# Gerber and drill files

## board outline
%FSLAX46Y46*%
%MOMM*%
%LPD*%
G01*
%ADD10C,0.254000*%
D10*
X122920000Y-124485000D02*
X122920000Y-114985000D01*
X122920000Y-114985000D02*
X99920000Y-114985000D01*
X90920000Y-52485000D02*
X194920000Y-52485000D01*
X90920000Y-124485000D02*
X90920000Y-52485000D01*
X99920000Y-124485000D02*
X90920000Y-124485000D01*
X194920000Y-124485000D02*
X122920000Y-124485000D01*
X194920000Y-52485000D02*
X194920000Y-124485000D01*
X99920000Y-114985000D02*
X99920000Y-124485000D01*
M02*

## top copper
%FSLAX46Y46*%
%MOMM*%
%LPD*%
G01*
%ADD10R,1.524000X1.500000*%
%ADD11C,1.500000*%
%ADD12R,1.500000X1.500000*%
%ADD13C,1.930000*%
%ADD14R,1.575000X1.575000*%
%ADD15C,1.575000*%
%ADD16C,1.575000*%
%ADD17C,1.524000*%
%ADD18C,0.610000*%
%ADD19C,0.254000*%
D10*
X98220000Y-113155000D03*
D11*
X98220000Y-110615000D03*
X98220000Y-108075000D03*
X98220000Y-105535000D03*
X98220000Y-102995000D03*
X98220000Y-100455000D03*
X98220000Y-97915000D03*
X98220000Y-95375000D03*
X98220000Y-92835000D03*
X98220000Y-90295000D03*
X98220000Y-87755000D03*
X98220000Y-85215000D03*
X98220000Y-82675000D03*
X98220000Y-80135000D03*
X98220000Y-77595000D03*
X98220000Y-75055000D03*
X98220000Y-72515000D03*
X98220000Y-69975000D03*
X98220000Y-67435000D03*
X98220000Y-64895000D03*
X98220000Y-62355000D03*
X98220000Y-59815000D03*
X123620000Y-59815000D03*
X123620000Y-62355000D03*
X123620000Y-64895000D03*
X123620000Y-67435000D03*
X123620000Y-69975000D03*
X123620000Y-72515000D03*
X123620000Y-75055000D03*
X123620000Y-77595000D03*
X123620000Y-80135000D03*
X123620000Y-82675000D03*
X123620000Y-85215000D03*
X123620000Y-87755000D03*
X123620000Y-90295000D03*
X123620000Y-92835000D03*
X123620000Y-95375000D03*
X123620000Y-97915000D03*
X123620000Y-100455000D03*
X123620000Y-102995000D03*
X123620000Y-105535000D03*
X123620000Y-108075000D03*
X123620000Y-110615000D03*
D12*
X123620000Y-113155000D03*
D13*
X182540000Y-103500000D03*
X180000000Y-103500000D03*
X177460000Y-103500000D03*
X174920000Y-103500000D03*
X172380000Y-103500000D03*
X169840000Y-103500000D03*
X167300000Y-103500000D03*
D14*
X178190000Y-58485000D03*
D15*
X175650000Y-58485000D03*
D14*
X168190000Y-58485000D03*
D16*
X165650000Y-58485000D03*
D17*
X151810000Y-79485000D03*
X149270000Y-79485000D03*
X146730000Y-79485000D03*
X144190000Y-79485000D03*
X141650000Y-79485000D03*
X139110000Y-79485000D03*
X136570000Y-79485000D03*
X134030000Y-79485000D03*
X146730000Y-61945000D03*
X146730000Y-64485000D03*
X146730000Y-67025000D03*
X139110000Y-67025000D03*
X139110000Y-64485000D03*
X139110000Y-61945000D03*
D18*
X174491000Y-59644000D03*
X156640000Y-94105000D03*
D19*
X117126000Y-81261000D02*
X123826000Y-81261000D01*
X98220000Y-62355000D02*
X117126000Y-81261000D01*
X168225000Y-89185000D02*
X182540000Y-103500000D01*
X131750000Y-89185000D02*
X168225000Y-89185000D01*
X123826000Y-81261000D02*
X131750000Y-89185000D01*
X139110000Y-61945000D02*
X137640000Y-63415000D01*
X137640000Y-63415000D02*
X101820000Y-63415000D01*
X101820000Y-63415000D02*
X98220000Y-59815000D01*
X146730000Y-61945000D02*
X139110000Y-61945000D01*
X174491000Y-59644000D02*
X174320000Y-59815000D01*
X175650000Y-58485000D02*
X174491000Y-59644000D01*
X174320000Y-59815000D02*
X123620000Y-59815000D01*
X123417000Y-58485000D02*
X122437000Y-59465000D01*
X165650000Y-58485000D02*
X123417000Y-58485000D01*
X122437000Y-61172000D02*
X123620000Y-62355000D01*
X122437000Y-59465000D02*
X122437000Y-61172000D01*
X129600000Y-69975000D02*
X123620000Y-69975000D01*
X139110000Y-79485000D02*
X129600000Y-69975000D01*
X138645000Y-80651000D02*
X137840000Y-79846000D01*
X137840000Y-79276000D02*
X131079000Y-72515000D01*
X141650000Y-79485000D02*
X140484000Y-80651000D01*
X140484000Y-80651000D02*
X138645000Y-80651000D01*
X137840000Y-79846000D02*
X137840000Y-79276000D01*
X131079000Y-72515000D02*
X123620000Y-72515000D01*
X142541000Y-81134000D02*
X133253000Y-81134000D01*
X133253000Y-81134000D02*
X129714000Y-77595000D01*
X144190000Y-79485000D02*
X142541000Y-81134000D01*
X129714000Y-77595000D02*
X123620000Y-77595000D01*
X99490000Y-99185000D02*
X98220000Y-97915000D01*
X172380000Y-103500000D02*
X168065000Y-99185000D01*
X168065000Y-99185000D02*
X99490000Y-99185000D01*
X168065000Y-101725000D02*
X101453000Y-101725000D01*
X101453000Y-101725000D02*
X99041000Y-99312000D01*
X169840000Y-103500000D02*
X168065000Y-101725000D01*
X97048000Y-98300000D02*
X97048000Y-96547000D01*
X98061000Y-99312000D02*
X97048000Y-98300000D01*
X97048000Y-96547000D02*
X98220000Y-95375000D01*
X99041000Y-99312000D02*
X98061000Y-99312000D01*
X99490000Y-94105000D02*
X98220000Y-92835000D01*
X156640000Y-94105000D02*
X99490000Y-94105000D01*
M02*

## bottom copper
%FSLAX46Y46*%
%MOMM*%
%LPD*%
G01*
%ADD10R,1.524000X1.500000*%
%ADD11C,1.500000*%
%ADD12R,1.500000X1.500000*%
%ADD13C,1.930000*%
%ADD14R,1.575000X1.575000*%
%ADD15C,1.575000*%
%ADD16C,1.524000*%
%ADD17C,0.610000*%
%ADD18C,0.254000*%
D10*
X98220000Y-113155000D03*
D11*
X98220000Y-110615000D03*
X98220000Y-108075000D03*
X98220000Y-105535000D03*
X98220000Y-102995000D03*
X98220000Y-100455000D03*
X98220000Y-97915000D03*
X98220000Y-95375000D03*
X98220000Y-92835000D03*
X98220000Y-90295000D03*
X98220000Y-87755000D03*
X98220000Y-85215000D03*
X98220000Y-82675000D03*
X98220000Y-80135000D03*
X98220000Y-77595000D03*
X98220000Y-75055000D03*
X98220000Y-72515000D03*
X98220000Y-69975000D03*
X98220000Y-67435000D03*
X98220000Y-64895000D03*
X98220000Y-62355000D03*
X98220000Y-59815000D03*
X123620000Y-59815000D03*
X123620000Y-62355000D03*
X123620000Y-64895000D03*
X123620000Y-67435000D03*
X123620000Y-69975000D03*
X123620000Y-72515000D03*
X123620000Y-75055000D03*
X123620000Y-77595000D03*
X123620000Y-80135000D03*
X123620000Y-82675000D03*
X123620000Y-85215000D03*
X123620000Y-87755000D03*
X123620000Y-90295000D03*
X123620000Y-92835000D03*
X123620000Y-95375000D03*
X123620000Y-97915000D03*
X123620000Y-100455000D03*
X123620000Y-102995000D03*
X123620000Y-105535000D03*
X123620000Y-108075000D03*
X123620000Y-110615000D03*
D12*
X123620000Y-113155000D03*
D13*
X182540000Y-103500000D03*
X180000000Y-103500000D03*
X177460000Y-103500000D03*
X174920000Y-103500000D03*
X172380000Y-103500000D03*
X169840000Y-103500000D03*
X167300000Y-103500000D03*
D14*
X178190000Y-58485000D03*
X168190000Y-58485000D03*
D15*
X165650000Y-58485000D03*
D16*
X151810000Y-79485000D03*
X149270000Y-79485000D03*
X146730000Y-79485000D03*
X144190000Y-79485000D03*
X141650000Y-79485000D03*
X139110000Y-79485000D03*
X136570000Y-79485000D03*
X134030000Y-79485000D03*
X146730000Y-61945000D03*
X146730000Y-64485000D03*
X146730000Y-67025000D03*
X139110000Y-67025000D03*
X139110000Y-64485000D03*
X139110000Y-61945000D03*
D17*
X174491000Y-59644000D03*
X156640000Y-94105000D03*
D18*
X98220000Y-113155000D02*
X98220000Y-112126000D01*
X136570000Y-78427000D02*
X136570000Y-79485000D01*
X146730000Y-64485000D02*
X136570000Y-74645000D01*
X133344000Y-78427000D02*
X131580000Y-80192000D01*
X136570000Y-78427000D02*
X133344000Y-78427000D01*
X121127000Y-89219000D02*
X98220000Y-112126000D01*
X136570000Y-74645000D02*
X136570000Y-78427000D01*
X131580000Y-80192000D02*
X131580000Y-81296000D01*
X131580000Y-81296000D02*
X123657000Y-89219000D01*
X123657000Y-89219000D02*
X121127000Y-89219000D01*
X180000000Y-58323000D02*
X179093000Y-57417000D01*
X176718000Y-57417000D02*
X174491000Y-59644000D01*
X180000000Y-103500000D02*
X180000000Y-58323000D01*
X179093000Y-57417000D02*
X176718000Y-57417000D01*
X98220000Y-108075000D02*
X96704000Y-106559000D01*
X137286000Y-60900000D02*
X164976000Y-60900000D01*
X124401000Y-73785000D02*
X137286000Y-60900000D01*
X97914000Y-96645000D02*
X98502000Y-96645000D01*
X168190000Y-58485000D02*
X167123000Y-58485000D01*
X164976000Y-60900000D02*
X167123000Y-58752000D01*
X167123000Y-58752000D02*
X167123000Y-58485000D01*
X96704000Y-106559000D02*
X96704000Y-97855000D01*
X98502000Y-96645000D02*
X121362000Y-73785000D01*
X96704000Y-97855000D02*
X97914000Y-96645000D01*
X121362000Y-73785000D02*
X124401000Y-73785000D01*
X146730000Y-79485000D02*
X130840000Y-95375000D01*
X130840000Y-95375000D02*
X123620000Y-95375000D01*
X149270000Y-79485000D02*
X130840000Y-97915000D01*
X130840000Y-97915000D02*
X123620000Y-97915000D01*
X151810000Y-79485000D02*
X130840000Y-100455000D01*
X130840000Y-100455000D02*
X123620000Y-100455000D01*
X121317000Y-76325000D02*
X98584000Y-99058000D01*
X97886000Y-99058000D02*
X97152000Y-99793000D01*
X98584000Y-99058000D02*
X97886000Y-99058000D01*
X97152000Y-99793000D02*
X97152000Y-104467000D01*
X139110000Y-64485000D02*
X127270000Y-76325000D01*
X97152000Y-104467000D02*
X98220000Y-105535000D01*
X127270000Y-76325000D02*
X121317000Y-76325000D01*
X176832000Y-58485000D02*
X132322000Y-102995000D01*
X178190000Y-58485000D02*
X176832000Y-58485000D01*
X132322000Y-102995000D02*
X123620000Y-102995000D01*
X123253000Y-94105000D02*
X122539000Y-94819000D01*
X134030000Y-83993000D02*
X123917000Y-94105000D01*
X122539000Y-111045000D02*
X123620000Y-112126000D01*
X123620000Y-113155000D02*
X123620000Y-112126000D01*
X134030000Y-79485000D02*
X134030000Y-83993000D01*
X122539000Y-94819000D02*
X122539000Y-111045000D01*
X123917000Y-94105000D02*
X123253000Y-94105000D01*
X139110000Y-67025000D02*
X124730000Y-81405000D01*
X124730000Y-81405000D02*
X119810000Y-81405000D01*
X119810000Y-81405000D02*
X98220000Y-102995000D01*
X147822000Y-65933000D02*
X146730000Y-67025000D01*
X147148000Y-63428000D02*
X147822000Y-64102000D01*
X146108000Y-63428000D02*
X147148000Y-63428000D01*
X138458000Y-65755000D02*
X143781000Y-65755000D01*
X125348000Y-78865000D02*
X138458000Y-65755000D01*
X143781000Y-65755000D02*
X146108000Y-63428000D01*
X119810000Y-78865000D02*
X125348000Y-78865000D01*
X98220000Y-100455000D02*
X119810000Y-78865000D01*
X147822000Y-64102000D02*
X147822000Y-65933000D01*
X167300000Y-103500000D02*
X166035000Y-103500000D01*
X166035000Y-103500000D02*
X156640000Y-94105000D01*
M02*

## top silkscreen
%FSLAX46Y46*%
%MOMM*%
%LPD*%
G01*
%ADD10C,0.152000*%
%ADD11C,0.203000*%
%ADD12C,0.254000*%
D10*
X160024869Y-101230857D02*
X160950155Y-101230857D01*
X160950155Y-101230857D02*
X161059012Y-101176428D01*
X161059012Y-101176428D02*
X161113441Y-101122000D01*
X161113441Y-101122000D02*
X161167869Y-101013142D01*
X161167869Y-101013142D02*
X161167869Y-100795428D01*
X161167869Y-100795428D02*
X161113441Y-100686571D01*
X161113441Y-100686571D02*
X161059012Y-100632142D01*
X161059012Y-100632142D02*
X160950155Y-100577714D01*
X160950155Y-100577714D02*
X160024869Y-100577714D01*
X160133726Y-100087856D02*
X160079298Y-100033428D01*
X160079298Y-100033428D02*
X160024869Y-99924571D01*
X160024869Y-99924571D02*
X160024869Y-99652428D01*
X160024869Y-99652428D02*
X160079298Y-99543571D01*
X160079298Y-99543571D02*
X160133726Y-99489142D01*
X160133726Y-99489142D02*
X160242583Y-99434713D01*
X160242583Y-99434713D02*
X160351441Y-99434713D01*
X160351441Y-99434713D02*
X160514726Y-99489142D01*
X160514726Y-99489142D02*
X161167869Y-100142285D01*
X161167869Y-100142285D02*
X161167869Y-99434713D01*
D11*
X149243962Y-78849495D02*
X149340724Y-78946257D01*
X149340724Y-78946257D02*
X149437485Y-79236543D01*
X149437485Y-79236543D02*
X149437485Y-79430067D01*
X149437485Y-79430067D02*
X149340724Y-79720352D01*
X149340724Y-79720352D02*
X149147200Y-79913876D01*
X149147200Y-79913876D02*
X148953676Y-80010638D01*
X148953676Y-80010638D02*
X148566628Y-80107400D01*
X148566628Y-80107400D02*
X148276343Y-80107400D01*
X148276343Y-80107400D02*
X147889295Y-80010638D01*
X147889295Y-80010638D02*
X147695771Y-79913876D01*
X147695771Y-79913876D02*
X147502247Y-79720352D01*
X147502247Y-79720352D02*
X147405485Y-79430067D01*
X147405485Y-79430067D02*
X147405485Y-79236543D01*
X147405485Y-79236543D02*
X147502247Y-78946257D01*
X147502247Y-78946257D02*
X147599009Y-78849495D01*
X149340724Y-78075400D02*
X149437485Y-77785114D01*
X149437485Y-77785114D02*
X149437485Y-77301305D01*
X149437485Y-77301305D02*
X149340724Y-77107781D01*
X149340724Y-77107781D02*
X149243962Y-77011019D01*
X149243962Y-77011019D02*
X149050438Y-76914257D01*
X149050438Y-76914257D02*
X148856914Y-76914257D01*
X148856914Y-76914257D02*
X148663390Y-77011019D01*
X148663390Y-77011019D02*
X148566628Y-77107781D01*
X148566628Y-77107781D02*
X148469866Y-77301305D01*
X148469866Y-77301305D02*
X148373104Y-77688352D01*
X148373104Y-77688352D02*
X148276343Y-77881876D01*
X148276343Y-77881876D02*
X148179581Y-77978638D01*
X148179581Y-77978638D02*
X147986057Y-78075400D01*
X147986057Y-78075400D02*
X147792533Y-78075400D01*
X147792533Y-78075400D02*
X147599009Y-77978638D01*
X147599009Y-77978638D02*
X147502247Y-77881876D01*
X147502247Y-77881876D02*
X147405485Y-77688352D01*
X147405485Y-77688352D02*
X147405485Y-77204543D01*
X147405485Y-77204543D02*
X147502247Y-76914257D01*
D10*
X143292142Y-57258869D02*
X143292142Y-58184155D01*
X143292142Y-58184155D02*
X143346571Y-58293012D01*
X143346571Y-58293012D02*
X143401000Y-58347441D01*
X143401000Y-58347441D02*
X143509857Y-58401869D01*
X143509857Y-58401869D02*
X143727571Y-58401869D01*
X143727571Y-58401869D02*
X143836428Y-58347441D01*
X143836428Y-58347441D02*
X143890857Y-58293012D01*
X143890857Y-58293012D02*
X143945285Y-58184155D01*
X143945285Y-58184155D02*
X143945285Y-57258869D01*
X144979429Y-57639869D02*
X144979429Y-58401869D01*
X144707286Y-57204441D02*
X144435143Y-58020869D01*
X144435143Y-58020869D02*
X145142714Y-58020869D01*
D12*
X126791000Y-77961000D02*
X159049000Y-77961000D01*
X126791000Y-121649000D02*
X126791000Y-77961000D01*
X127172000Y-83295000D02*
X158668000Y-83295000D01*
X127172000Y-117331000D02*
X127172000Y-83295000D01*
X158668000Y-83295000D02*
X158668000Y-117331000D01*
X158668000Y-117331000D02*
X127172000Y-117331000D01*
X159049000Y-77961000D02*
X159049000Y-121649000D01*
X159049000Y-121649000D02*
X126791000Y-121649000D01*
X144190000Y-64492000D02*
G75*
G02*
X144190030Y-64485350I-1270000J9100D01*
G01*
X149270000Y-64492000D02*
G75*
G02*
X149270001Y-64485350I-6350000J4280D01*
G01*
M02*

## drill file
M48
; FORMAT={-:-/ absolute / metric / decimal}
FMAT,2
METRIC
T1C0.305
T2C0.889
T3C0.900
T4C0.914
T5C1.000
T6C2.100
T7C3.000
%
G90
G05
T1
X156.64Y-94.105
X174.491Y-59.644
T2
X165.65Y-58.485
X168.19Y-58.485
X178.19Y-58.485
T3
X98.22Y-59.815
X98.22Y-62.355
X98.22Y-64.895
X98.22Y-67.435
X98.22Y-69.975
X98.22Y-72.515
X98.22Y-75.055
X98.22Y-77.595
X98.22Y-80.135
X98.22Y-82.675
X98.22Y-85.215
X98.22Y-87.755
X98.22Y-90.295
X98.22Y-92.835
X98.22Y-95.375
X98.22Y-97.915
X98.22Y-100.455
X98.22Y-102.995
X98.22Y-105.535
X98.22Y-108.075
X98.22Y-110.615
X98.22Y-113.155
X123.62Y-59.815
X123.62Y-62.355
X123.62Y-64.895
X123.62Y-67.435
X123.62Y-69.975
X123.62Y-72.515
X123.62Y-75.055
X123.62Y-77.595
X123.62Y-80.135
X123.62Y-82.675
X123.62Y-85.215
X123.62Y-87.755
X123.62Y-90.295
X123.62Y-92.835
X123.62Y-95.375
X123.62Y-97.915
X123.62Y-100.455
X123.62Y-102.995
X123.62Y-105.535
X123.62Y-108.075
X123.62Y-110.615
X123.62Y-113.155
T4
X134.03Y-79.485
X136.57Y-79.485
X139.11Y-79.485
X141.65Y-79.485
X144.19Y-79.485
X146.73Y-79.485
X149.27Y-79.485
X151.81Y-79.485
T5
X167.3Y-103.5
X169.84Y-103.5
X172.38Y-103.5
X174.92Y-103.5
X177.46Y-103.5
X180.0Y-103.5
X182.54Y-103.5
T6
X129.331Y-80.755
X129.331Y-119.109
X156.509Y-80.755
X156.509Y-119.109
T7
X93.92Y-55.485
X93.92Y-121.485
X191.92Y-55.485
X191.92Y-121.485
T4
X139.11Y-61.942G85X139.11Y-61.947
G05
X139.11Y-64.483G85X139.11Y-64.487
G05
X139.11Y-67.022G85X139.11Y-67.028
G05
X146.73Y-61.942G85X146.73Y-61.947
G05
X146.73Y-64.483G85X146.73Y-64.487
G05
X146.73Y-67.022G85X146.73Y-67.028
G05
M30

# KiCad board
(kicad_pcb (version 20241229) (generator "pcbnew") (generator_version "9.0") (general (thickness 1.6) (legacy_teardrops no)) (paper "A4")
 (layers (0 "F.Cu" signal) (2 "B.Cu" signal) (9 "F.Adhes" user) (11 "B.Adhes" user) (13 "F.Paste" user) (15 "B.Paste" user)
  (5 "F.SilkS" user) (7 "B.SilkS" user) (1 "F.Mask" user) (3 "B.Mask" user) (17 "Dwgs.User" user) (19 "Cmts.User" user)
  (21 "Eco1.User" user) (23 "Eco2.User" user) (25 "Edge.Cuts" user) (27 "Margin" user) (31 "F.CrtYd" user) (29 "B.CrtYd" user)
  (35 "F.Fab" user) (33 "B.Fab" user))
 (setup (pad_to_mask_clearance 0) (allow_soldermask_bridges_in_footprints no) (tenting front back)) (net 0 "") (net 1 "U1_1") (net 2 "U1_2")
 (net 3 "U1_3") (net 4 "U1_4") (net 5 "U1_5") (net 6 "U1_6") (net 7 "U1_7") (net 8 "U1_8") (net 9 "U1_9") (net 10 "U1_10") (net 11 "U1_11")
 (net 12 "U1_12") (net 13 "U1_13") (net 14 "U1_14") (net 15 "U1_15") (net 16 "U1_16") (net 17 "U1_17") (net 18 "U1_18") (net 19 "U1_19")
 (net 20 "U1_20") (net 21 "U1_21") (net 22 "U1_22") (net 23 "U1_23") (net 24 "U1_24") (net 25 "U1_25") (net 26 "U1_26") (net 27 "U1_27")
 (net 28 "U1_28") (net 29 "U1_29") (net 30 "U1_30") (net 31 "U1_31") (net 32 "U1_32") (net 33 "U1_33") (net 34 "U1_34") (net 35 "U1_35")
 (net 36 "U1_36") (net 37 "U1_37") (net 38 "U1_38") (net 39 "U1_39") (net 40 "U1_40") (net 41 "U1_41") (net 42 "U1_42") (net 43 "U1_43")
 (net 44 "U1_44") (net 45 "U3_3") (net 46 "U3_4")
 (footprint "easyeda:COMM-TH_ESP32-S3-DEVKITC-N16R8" (layer "F.Cu") (at 110.92 86.485 180)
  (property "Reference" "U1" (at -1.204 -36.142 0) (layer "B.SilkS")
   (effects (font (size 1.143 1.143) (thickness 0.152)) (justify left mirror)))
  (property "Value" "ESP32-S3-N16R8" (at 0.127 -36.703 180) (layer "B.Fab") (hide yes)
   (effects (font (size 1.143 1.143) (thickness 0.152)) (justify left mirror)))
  (pad "1" thru_hole rect (at 12.7 -26.67 180) (size 1.524 1.5) (drill 0.9) (layers "*.Cu" "*.Paste" "*.Mask") (remove_unused_layers no)
   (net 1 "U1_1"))
  (pad "2" thru_hole circle (at 12.7 -24.13 180) (size 1.5 1.5) (drill 0.9) (layers "*.Cu" "*.Paste" "*.Mask") (remove_unused_layers no)
   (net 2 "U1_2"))
  (pad "3" thru_hole circle (at 12.7 -21.59 180) (size 1.5 1.5) (drill 0.9) (layers "*.Cu" "*.Paste" "*.Mask") (remove_unused_layers no)
   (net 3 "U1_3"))
  (pad "4" thru_hole circle (at 12.7 -19.05 180) (size 1.5 1.5) (drill 0.9) (layers "*.Cu" "*.Paste" "*.Mask") (remove_unused_layers no)
   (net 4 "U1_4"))
  (pad "5" thru_hole circle (at 12.7 -16.51 180) (size 1.5 1.5) (drill 0.9) (layers "*.Cu" "*.Paste" "*.Mask") (remove_unused_layers no)
   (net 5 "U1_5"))
  (pad "6" thru_hole circle (at 12.7 -13.97 180) (size 1.5 1.5) (drill 0.9) (layers "*.Cu" "*.Paste" "*.Mask") (remove_unused_layers no)
   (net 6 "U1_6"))
  (pad "7" thru_hole circle (at 12.7 -11.43 180) (size 1.5 1.5) (drill 0.9) (layers "*.Cu" "*.Paste" "*.Mask") (remove_unused_layers no)
   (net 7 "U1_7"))
  (pad "8" thru_hole circle (at 12.7 -8.89 180) (size 1.5 1.5) (drill 0.9) (layers "*.Cu" "*.Paste" "*.Mask") (remove_unused_layers no)
   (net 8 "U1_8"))
  (pad "9" thru_hole circle (at 12.7 -6.35 180) (size 1.5 1.5) (drill 0.9) (layers "*.Cu" "*.Paste" "*.Mask") (remove_unused_layers no)
   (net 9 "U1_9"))
  (pad "10" thru_hole circle (at 12.7 -3.81 180) (size 1.5 1.5) (drill 0.9) (layers "*.Cu" "*.Paste" "*.Mask") (remove_unused_layers no)
   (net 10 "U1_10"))
  (pad "11" thru_hole circle (at 12.7 -1.27 180) (size 1.5 1.5) (drill 0.9) (layers "*.Cu" "*.Paste" "*.Mask") (remove_unused_layers no)
   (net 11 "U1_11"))
  (pad "12" thru_hole circle (at 12.7 1.27 180) (size 1.5 1.5) (drill 0.9) (layers "*.Cu" "*.Paste" "*.Mask") (remove_unused_layers no)
   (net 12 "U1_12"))
  (pad "13" thru_hole circle (at 12.7 3.81 180) (size 1.5 1.5) (drill 0.9) (layers "*.Cu" "*.Paste" "*.Mask") (remove_unused_layers no)
   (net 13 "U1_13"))
  (pad "14" thru_hole circle (at 12.7 6.35 180) (size 1.5 1.5) (drill 0.9) (layers "*.Cu" "*.Paste" "*.Mask") (remove_unused_layers no)
   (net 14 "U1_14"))
  (pad "15" thru_hole circle (at 12.7 8.89 180) (size 1.5 1.5) (drill 0.9) (layers "*.Cu" "*.Paste" "*.Mask") (remove_unused_layers no)
   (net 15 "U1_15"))
  (pad "16" thru_hole circle (at 12.7 11.43 180) (size 1.5 1.5) (drill 0.9) (layers "*.Cu" "*.Paste" "*.Mask") (remove_unused_layers no)
   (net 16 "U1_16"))
  (pad "17" thru_hole circle (at 12.7 13.97 180) (size 1.5 1.5) (drill 0.9) (layers "*.Cu" "*.Paste" "*.Mask") (remove_unused_layers no)
   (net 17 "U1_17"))
  (pad "18" thru_hole circle (at 12.7 16.51 180) (size 1.5 1.5) (drill 0.9) (layers "*.Cu" "*.Paste" "*.Mask") (remove_unused_layers no)
   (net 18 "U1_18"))
  (pad "19" thru_hole circle (at 12.7 19.05 180) (size 1.5 1.5) (drill 0.9) (layers "*.Cu" "*.Paste" "*.Mask") (remove_unused_layers no)
   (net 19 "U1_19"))
  (pad "20" thru_hole circle (at 12.7 21.59 180) (size 1.5 1.5) (drill 0.9) (layers "*.Cu" "*.Paste" "*.Mask") (remove_unused_layers no)
   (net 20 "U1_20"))
  (pad "21" thru_hole circle (at 12.7 24.13 180) (size 1.5 1.5) (drill 0.9) (layers "*.Cu" "*.Paste" "*.Mask") (remove_unused_layers no)
   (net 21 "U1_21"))
  (pad "22" thru_hole circle (at 12.7 26.67 180) (size 1.5 1.5) (drill 0.9) (layers "*.Cu" "*.Paste" "*.Mask") (remove_unused_layers no)
   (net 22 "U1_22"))
  (pad "23" thru_hole circle (at -12.7 26.67 180) (size 1.5 1.5) (drill 0.9) (layers "*.Cu" "*.Paste" "*.Mask") (remove_unused_layers no)
   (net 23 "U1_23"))
  (pad "24" thru_hole circle (at -12.7 24.13 180) (size 1.5 1.5) (drill 0.9) (layers "*.Cu" "*.Paste" "*.Mask") (remove_unused_layers no)
   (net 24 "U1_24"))
  (pad "25" thru_hole circle (at -12.7 21.59 180) (size 1.5 1.5) (drill 0.9) (layers "*.Cu" "*.Paste" "*.Mask") (remove_unused_layers no)
   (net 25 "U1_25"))
  (pad "26" thru_hole circle (at -12.7 19.05 180) (size 1.5 1.5) (drill 0.9) (layers "*.Cu" "*.Paste" "*.Mask") (remove_unused_layers no)
   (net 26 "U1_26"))
  (pad "27" thru_hole circle (at -12.7 16.51 180) (size 1.5 1.5) (drill 0.9) (layers "*.Cu" "*.Paste" "*.Mask") (remove_unused_layers no)
   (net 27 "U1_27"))
  (pad "28" thru_hole circle (at -12.7 13.97 180) (size 1.5 1.5) (drill 0.9) (layers "*.Cu" "*.Paste" "*.Mask") (remove_unused_layers no)
   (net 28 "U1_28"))
  (pad "29" thru_hole circle (at -12.7 11.43 180) (size 1.5 1.5) (drill 0.9) (layers "*.Cu" "*.Paste" "*.Mask") (remove_unused_layers no)
   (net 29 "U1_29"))
  (pad "30" thru_hole circle (at -12.7 8.89 180) (size 1.5 1.5) (drill 0.9) (layers "*.Cu" "*.Paste" "*.Mask") (remove_unused_layers no)
   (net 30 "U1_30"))
  (pad "31" thru_hole circle (at -12.7 6.35 180) (size 1.5 1.5) (drill 0.9) (layers "*.Cu" "*.Paste" "*.Mask") (remove_unused_layers no)
   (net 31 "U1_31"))
  (pad "32" thru_hole circle (at -12.7 3.81 180) (size 1.5 1.5) (drill 0.9) (layers "*.Cu" "*.Paste" "*.Mask") (remove_unused_layers no)
   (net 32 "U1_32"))
  (pad "33" thru_hole circle (at -12.7 1.27 180) (size 1.5 1.5) (drill 0.9) (layers "*.Cu" "*.Paste" "*.Mask") (remove_unused_layers no)
   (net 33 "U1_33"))
  (pad "34" thru_hole circle (at -12.7 -1.27 180) (size 1.5 1.5) (drill 0.9) (layers "*.Cu" "*.Paste" "*.Mask") (remove_unused_layers no)
   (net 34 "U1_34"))
  (pad "35" thru_hole circle (at -12.7 -3.81 180) (size 1.5 1.5) (drill 0.9) (layers "*.Cu" "*.Paste" "*.Mask") (remove_unused_layers no)
   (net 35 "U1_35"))
  (pad "36" thru_hole circle (at -12.7 -6.35 180) (size 1.5 1.5) (drill 0.9) (layers "*.Cu" "*.Paste" "*.Mask") (remove_unused_layers no)
   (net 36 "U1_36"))
  (pad "37" thru_hole circle (at -12.7 -8.89 180) (size 1.5 1.5) (drill 0.9) (layers "*.Cu" "*.Paste" "*.Mask") (remove_unused_layers no)
   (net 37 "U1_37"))
  (pad "38" thru_hole circle (at -12.7 -11.43 180) (size 1.5 1.5) (drill 0.9) (layers "*.Cu" "*.Paste" "*.Mask") (remove_unused_layers no)
   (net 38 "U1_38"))
  (pad "39" thru_hole circle (at -12.7 -13.97 180) (size 1.5 1.5) (drill 0.9) (layers "*.Cu" "*.Paste" "*.Mask") (remove_unused_layers no)
   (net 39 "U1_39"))
  (pad "40" thru_hole circle (at -12.7 -16.51 180) (size 1.5 1.5) (drill 0.9) (layers "*.Cu" "*.Paste" "*.Mask") (remove_unused_layers no)
   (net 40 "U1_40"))
  (pad "41" thru_hole circle (at -12.7 -19.05 180) (size 1.5 1.5) (drill 0.9) (layers "*.Cu" "*.Paste" "*.Mask") (remove_unused_layers no)
   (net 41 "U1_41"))
  (pad "42" thru_hole circle (at -12.7 -21.59 180) (size 1.5 1.5) (drill 0.9) (layers "*.Cu" "*.Paste" "*.Mask") (remove_unused_layers no)
   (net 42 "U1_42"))
  (pad "43" thru_hole circle (at -12.7 -24.13 180) (size 1.5 1.5) (drill 0.9) (layers "*.Cu" "*.Paste" "*.Mask") (remove_unused_layers no)
   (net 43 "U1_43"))
  (pad "44" thru_hole rect (at -12.7 -26.67 180) (size 1.5 1.5) (drill 0.9) (layers "*.Cu" "*.Paste" "*.Mask") (remove_unused_layers no)
   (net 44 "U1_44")))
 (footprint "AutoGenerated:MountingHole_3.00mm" (layer "F.Cu") (at 93.92 55.485)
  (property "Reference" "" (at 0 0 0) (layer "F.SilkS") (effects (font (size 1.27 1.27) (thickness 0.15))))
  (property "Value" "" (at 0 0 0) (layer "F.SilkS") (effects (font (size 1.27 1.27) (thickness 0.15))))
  (pad "" np_thru_hole circle (at 0 0) (size 3 3) (drill 3) (layers "*.Cu" "*.Mask")))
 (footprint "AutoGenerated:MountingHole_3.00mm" (layer "F.Cu") (at 191.92 55.485)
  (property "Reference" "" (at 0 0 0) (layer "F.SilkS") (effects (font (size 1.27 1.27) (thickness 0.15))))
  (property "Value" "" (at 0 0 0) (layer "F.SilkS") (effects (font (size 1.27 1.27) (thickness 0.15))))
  (pad "" np_thru_hole circle (at 0 0) (size 3 3) (drill 3) (layers "*.Cu" "*.Mask")))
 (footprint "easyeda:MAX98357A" (layer "F.Cu") (at 174.92 110.485 90)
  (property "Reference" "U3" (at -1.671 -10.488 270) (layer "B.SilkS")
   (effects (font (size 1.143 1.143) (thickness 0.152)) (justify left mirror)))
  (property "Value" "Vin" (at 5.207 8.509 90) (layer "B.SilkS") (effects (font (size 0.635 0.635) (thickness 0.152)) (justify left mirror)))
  (pad "1" thru_hole circle (at 6.985 7.62 270) (size 1.93 1.93) (drill oval 1) (layers "*.Cu" "*.Paste" "*.Mask") (remove_unused_layers no)
   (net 21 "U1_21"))
  (pad "2" thru_hole circle (at 6.985 5.08 270) (size 1.93 1.93) (drill oval 1) (layers "*.Cu" "*.Paste" "*.Mask") (remove_unused_layers no)
   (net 23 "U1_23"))
  (pad "3" thru_hole circle (at 6.985 2.54 270) (size 1.93 1.93) (drill oval 1) (layers "*.Cu" "*.Paste" "*.Mask") (remove_unused_layers no)
   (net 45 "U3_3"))
  (pad "4" thru_hole circle (at 6.985 0 270) (size 1.93 1.93) (drill oval 1) (layers "*.Cu" "*.Paste" "*.Mask") (remove_unused_layers no)
   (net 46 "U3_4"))
  (pad "5" thru_hole circle (at 6.985 -2.54 270) (size 1.93 1.93) (drill oval 1) (layers "*.Cu" "*.Paste" "*.Mask")
   (remove_unused_layers no) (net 7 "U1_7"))
  (pad "6" thru_hole circle (at 6.985 -5.08 270) (size 1.93 1.93) (drill oval 1) (layers "*.Cu" "*.Paste" "*.Mask")
   (remove_unused_layers no) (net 8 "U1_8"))
  (pad "7" thru_hole circle (at 6.985 -7.62 270) (size 1.93 1.93) (drill oval 1) (layers "*.Cu" "*.Paste" "*.Mask")
   (remove_unused_layers no) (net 9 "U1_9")))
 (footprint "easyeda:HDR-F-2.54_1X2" (layer "F.Cu") (at 176.92 58.485)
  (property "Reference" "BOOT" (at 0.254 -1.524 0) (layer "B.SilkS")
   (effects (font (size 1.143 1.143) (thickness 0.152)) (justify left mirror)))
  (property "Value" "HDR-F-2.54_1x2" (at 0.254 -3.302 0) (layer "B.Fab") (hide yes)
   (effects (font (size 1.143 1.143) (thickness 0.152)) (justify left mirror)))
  (pad "1" thru_hole rect (at 1.27 0 90) (size 1.575 1.575) (drill 0.889) (layers "*.Cu" "*.Paste" "*.Mask") (remove_unused_layers no)
   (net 40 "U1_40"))
  (pad "2" smd circle (at -1.27 0 90) (size 1.575 1.575) (layers "F.Cu" "F.Mask" "F.Paste") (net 23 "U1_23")))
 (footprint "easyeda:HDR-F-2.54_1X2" (layer "F.Cu") (at 166.92 58.485)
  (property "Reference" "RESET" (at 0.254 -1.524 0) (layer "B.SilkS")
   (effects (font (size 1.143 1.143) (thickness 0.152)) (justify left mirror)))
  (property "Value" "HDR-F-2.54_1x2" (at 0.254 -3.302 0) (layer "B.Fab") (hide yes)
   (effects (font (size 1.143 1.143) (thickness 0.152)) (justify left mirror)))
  (pad "1" thru_hole rect (at 1.27 0 90) (size 1.575 1.575) (drill 0.889) (layers "*.Cu" "*.Paste" "*.Mask") (remove_unused_layers no)
   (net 3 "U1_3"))
  (pad "2" thru_hole circle (at -1.27 0 90) (size 1.575 1.575) (drill 0.889) (layers "*.Cu" "*.Paste" "*.Mask") (remove_unused_layers no)
   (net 24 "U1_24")))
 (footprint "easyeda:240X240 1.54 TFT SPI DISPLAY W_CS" (layer "F.Cu") (at 142.92 79.485 -90)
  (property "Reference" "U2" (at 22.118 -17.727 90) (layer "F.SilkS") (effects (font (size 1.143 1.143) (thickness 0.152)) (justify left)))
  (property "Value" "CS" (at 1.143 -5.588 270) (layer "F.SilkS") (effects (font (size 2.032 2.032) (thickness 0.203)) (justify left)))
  (fp_line (start -1.524 16.129) (end -1.524 -16.129) (stroke (width 0.254) (type solid)) (layer "F.SilkS"))
  (fp_line (start 42.164 16.129) (end -1.524 16.129) (stroke (width 0.254) (type solid)) (layer "F.SilkS"))
  (fp_line (start 3.81 15.748) (end 3.81 -15.748) (stroke (width 0.254) (type solid)) (layer "F.SilkS"))
  (fp_line (start 37.846 15.748) (end 3.81 15.748) (stroke (width 0.254) (type solid)) (layer "F.SilkS"))
  (fp_line (start 3.81 -15.748) (end 37.846 -15.748) (stroke (width 0.254) (type solid)) (layer "F.SilkS"))
  (fp_line (start 37.846 -15.748) (end 37.846 15.748) (stroke (width 0.254) (type solid)) (layer "F.SilkS"))
  (fp_line (start -1.524 -16.129) (end 42.164 -16.129) (stroke (width 0.254) (type solid)) (layer "F.SilkS"))
  (fp_line (start 42.164 -16.129) (end 42.164 16.129) (stroke (width 0.254) (type solid)) (layer "F.SilkS"))
  (pad "" np_thru_hole circle (at 1.27 -13.589) (size 2.1 2.1) (drill 2.1) (layers "*.Cu" "*.Mask"))
  (pad "" np_thru_hole circle (at 1.27 13.589) (size 2.1 2.1) (drill 2.1) (layers "*.Cu" "*.Mask"))
  (pad "" np_thru_hole circle (at 39.624 -13.589) (size 2.1 2.1) (drill 2.1) (layers "*.Cu" "*.Mask"))
  (pad "" np_thru_hole circle (at 39.624 13.589) (size 2.1 2.1) (drill 2.1) (layers "*.Cu" "*.Mask"))
  (pad "1" thru_hole circle (at 0 -8.89 270) (size 1.524 1.524) (drill 0.914) (layers "*.Cu" "*.Paste" "*.Mask") (remove_unused_layers no)
   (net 39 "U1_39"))
  (pad "2" thru_hole circle (at 0 -6.35 270) (size 1.524 1.524) (drill 0.914) (layers "*.Cu" "*.Paste" "*.Mask") (remove_unused_layers no)
   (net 38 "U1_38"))
  (pad "3" thru_hole circle (at 0 -3.81 270) (size 1.524 1.524) (drill 0.914) (layers "*.Cu" "*.Paste" "*.Mask") (remove_unused_layers no)
   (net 37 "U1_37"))
  (pad "4" thru_hole circle (at 0 -1.27 270) (size 1.524 1.524) (drill 0.914) (layers "*.Cu" "*.Paste" "*.Mask") (remove_unused_layers no)
   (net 30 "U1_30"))
  (pad "5" thru_hole circle (at 0 1.27 270) (size 1.524 1.524) (drill 0.914) (layers "*.Cu" "*.Paste" "*.Mask") (remove_unused_layers no)
   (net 28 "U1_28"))
  (pad "6" thru_hole circle (at 0 3.81 270) (size 1.524 1.524) (drill 0.914) (layers "*.Cu" "*.Paste" "*.Mask") (remove_unused_layers no)
   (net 27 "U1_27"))
  (pad "7" thru_hole circle (at 0 6.35 270) (size 1.524 1.524) (drill 0.914) (layers "*.Cu" "*.Paste" "*.Mask") (remove_unused_layers no)
   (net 1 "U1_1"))
  (pad "8" thru_hole circle (at 0 8.89 270) (size 1.524 1.524) (drill 0.914) (layers "*.Cu" "*.Paste" "*.Mask") (remove_unused_layers no)
   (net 44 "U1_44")))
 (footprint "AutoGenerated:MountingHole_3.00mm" (layer "F.Cu") (at 191.92 121.485)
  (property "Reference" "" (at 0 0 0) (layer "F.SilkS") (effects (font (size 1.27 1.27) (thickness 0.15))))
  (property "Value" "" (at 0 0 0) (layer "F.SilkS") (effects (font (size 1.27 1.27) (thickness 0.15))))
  (pad "" np_thru_hole circle (at 0 0) (size 3 3) (drill 3) (layers "*.Cu" "*.Mask")))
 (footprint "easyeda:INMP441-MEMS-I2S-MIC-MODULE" (layer "F.Cu") (at 142.92 64.485)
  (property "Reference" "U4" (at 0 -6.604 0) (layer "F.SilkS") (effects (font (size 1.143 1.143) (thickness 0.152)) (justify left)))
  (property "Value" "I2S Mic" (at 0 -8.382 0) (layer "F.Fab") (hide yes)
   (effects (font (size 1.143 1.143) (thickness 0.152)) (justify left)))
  (fp_arc (start 1.27 0.007) (mid -1.270019 -0.007675) (end 1.27003 0.00035) (stroke (width 0.254) (type solid)) (layer "F.SilkS"))
  (fp_arc (start 6.35 0.007) (mid -6.350001 0.002325) (end 6.350001 0.00035) (stroke (width 0.254) (type solid)) (layer "F.SilkS"))
  (pad "1" thru_hole circle (at 3.81 -2.54) (size 1.524 1.524) (drill oval 0.914 0.919) (layers "*.Cu" "*.Paste" "*.Mask")
   (remove_unused_layers no) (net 22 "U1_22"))
  (pad "2" thru_hole circle (at 3.81 0) (size 1.524 1.524) (drill oval 0.914 0.919) (layers "*.Cu" "*.Paste" "*.Mask")
   (remove_unused_layers no) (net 1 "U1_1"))
  (pad "3" thru_hole circle (at 3.81 2.54) (size 1.524 1.524) (drill oval 0.914 0.919) (layers "*.Cu" "*.Paste" "*.Mask")
   (remove_unused_layers no) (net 6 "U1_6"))
  (pad "4" thru_hole circle (at -3.81 2.54) (size 1.524 1.524) (drill oval 0.914 0.919) (layers "*.Cu" "*.Paste" "*.Mask")
   (remove_unused_layers no) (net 5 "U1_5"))
  (pad "5" thru_hole circle (at -3.81 0) (size 1.524 1.524) (drill oval 0.914 0.919) (layers "*.Cu" "*.Paste" "*.Mask")
   (remove_unused_layers no) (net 4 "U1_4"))
  (pad "6" thru_hole circle (at -3.81 -2.54) (size 1.524 1.524) (drill oval 0.914 0.919) (layers "*.Cu" "*.Paste" "*.Mask")
   (remove_unused_layers no) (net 22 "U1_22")))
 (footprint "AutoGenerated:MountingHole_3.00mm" (layer "F.Cu") (at 93.92 121.485)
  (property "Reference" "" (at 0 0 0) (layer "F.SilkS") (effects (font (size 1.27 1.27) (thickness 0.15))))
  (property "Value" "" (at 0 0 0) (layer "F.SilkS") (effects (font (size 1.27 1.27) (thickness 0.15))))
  (pad "" np_thru_hole circle (at 0 0) (size 3 3) (drill 3) (layers "*.Cu" "*.Mask")))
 (gr_line (start 122.92 124.485) (end 122.92 114.985) (stroke (width 0.254) (type solid)) (layer "Edge.Cuts"))
 (gr_line (start 122.92 114.985) (end 99.92 114.985) (stroke (width 0.254) (type solid)) (layer "Edge.Cuts"))
 (gr_line (start 90.92 52.485) (end 194.92 52.485) (stroke (width 0.254) (type solid)) (layer "Edge.Cuts"))
 (gr_line (start 90.92 124.485) (end 90.92 52.485) (stroke (width 0.254) (type solid)) (layer "Edge.Cuts"))
 (gr_line (start 99.92 124.485) (end 90.92 124.485) (stroke (width 0.254) (type solid)) (layer "Edge.Cuts"))
 (gr_line (start 194.92 124.485) (end 122.92 124.485) (stroke (width 0.254) (type solid)) (layer "Edge.Cuts"))
 (gr_line (start 194.92 52.485) (end 194.92 124.485) (stroke (width 0.254) (type solid)) (layer "Edge.Cuts"))
 (gr_line (start 99.92 114.985) (end 99.92 124.485) (stroke (width 0.254) (type solid)) (layer "Edge.Cuts"))
 (segment (start 98.22 113.155) (end 98.22 112.126) (width 0.254) (layer "B.Cu") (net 1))
 (segment (start 136.57 78.427) (end 136.57 79.485) (width 0.254) (layer "B.Cu") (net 1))
 (segment (start 146.73 64.485) (end 136.57 74.645) (width 0.254) (layer "B.Cu") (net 1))
 (segment (start 133.344 78.427) (end 131.58 80.192) (width 0.254) (layer "B.Cu") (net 1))
 (segment (start 136.57 78.427) (end 133.344 78.427) (width 0.254) (layer "B.Cu") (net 1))
 (segment (start 121.127 89.219) (end 98.22 112.126) (width 0.254) (layer "B.Cu") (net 1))
 (segment (start 136.57 74.645) (end 136.57 78.427) (width 0.254) (layer "B.Cu") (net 1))
 (segment (start 131.58 80.192) (end 131.58 81.296) (width 0.254) (layer "B.Cu") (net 1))
 (segment (start 131.58 81.296) (end 123.657 89.219) (width 0.254) (layer "B.Cu") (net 1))
 (segment (start 123.657 89.219) (end 121.127 89.219) (width 0.254) (layer "B.Cu") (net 1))
 (segment (start 117.126 81.261) (end 123.826 81.261) (width 0.254) (layer "F.Cu") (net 21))
 (segment (start 98.22 62.355) (end 117.126 81.261) (width 0.254) (layer "F.Cu") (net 21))
 (segment (start 168.225 89.185) (end 182.54 103.5) (width 0.254) (layer "F.Cu") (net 21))
 (segment (start 131.75 89.185) (end 168.225 89.185) (width 0.254) (layer "F.Cu") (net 21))
 (segment (start 123.826 81.261) (end 131.75 89.185) (width 0.254) (layer "F.Cu") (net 21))
 (segment (start 139.11 61.945) (end 137.64 63.415) (width 0.254) (layer "F.Cu") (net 22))
 (segment (start 137.64 63.415) (end 101.82 63.415) (width 0.254) (layer "F.Cu") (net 22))
 (segment (start 101.82 63.415) (end 98.22 59.815) (width 0.254) (layer "F.Cu") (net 22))
 (segment (start 146.73 61.945) (end 139.11 61.945) (width 0.254) (layer "F.Cu") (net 22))
 (segment (start 174.491 59.644) (end 174.32 59.815) (width 0.254) (layer "F.Cu") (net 23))
 (segment (start 175.65 58.485) (end 174.491 59.644) (width 0.254) (layer "F.Cu") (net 23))
 (segment (start 174.32 59.815) (end 123.62 59.815) (width 0.254) (layer "F.Cu") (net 23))
 (via (at 174.491 59.644) (size 0.61) (drill 0.305) (layers "F.Cu" "B.Cu") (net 23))
 (segment (start 180 58.323) (end 179.093 57.417) (width 0.254) (layer "B.Cu") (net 23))
 (segment (start 176.718 57.417) (end 174.491 59.644) (width 0.254) (layer "B.Cu") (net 23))
 (segment (start 180 103.5) (end 180 58.323) (width 0.254) (layer "B.Cu") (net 23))
 (segment (start 179.093 57.417) (end 176.718 57.417) (width 0.254) (layer "B.Cu") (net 23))
 (segment (start 123.417 58.485) (end 122.437 59.465) (width 0.254) (layer "F.Cu") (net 24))
 (segment (start 165.65 58.485) (end 123.417 58.485) (width 0.254) (layer "F.Cu") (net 24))
 (segment (start 122.437 61.172) (end 123.62 62.355) (width 0.254) (layer "F.Cu") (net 24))
 (segment (start 122.437 59.465) (end 122.437 61.172) (width 0.254) (layer "F.Cu") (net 24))
 (segment (start 129.6 69.975) (end 123.62 69.975) (width 0.254) (layer "F.Cu") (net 27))
 (segment (start 139.11 79.485) (end 129.6 69.975) (width 0.254) (layer "F.Cu") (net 27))
 (segment (start 138.645 80.651) (end 137.84 79.846) (width 0.254) (layer "F.Cu") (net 28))
 (segment (start 137.84 79.276) (end 131.079 72.515) (width 0.254) (layer "F.Cu") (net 28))
 (segment (start 141.65 79.485) (end 140.484 80.651) (width 0.254) (layer "F.Cu") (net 28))
 (segment (start 140.484 80.651) (end 138.645 80.651) (width 0.254) (layer "F.Cu") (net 28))
 (segment (start 137.84 79.846) (end 137.84 79.276) (width 0.254) (layer "F.Cu") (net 28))
 (segment (start 131.079 72.515) (end 123.62 72.515) (width 0.254) (layer "F.Cu") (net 28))
 (segment (start 98.22 108.075) (end 96.704 106.559) (width 0.254) (layer "B.Cu") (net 3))
 (segment (start 137.286 60.9) (end 164.976 60.9) (width 0.254) (layer "B.Cu") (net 3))
 (segment (start 124.401 73.785) (end 137.286 60.9) (width 0.254) (layer "B.Cu") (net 3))
 (segment (start 97.914 96.645) (end 98.502 96.645) (width 0.254) (layer "B.Cu") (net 3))
 (segment (start 168.19 58.485) (end 167.123 58.485) (width 0.254) (layer "B.Cu") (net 3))
 (segment (start 164.976 60.9) (end 167.123 58.752) (width 0.254) (layer "B.Cu") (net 3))
 (segment (start 167.123 58.752) (end 167.123 58.485) (width 0.254) (layer "B.Cu") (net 3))
 (segment (start 96.704 106.559) (end 96.704 97.855) (width 0.254) (layer "B.Cu") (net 3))
 (segment (start 98.502 96.645) (end 121.362 73.785) (width 0.254) (layer "B.Cu") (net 3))
 (segment (start 96.704 97.855) (end 97.914 96.645) (width 0.254) (layer "B.Cu") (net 3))
 (segment (start 121.362 73.785) (end 124.401 73.785) (width 0.254) (layer "B.Cu") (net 3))
 (segment (start 142.541 81.134) (end 133.253 81.134) (width 0.254) (layer "F.Cu") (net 30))
 (segment (start 133.253 81.134) (end 129.714 77.595) (width 0.254) (layer "F.Cu") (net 30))
 (segment (start 144.19 79.485) (end 142.541 81.134) (width 0.254) (layer "F.Cu") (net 30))
 (segment (start 129.714 77.595) (end 123.62 77.595) (width 0.254) (layer "F.Cu") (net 30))
 (segment (start 146.73 79.485) (end 130.84 95.375) (width 0.254) (layer "B.Cu") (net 37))
 (segment (start 130.84 95.375) (end 123.62 95.375) (width 0.254) (layer "B.Cu") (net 37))
 (segment (start 149.27 79.485) (end 130.84 97.915) (width 0.254) (layer "B.Cu") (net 38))
 (segment (start 130.84 97.915) (end 123.62 97.915) (width 0.254) (layer "B.Cu") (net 38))
 (segment (start 151.81 79.485) (end 130.84 100.455) (width 0.254) (layer "B.Cu") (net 39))
 (segment (start 130.84 100.455) (end 123.62 100.455) (width 0.254) (layer "B.Cu") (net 39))
 (segment (start 121.317 76.325) (end 98.584 99.058) (width 0.254) (layer "B.Cu") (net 4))
 (segment (start 97.886 99.058) (end 97.152 99.793) (width 0.254) (layer "B.Cu") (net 4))
 (segment (start 98.584 99.058) (end 97.886 99.058) (width 0.254) (layer "B.Cu") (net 4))
 (segment (start 97.152 99.793) (end 97.152 104.467) (width 0.254) (layer "B.Cu") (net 4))
 (segment (start 139.11 64.485) (end 127.27 76.325) (width 0.254) (layer "B.Cu") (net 4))
 (segment (start 97.152 104.467) (end 98.22 105.535) (width 0.254) (layer "B.Cu") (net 4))
 (segment (start 127.27 76.325) (end 121.317 76.325) (width 0.254) (layer "B.Cu") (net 4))
 (segment (start 176.832 58.485) (end 132.322 102.995) (width 0.254) (layer "B.Cu") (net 40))
 (segment (start 178.19 58.485) (end 176.832 58.485) (width 0.254) (layer "B.Cu") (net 40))
 (segment (start 132.322 102.995) (end 123.62 102.995) (width 0.254) (layer "B.Cu") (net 40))
 (segment (start 123.253 94.105) (end 122.539 94.819) (width 0.254) (layer "B.Cu") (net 44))
 (segment (start 134.03 83.993) (end 123.917 94.105) (width 0.254) (layer "B.Cu") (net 44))
 (segment (start 122.539 111.045) (end 123.62 112.126) (width 0.254) (layer "B.Cu") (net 44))
 (segment (start 123.62 113.155) (end 123.62 112.126) (width 0.254) (layer "B.Cu") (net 44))
 (segment (start 134.03 79.485) (end 134.03 83.993) (width 0.254) (layer "B.Cu") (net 44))
 (segment (start 122.539 94.819) (end 122.539 111.045) (width 0.254) (layer "B.Cu") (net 44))
 (segment (start 123.917 94.105) (end 123.253 94.105) (width 0.254) (layer "B.Cu") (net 44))
 (segment (start 139.11 67.025) (end 124.73 81.405) (width 0.254) (layer "B.Cu") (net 5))
 (segment (start 124.73 81.405) (end 119.81 81.405) (width 0.254) (layer "B.Cu") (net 5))
 (segment (start 119.81 81.405) (end 98.22 102.995) (width 0.254) (layer "B.Cu") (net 5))
 (segment (start 147.822 65.933) (end 146.73 67.025) (width 0.254) (layer "B.Cu") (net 6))
 (segment (start 147.148 63.428) (end 147.822 64.102) (width 0.254) (layer "B.Cu") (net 6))
 (segment (start 146.108 63.428) (end 147.148 63.428) (width 0.254) (layer "B.Cu") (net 6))
 (segment (start 138.458 65.755) (end 143.781 65.755) (width 0.254) (layer "B.Cu") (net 6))
 (segment (start 125.348 78.865) (end 138.458 65.755) (width 0.254) (layer "B.Cu") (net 6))
 (segment (start 143.781 65.755) (end 146.108 63.428) (width 0.254) (layer "B.Cu") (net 6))
 (segment (start 119.81 78.865) (end 125.348 78.865) (width 0.254) (layer "B.Cu") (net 6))
 (segment (start 98.22 100.455) (end 119.81 78.865) (width 0.254) (layer "B.Cu") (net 6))
 (segment (start 147.822 64.102) (end 147.822 65.933) (width 0.254) (layer "B.Cu") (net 6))
 (segment (start 99.49 99.185) (end 98.22 97.915) (width 0.254) (layer "F.Cu") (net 7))
 (segment (start 172.38 103.5) (end 168.065 99.185) (width 0.254) (layer "F.Cu") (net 7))
 (segment (start 168.065 99.185) (end 99.49 99.185) (width 0.254) (layer "F.Cu") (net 7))
 (segment (start 168.065 101.725) (end 101.453 101.725) (width 0.254) (layer "F.Cu") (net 8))
 (segment (start 101.453 101.725) (end 99.041 99.312) (width 0.254) (layer "F.Cu") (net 8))
 (segment (start 169.84 103.5) (end 168.065 101.725) (width 0.254) (layer "F.Cu") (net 8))
 (segment (start 97.048 98.3) (end 97.048 96.547) (width 0.254) (layer "F.Cu") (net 8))
 (segment (start 98.061 99.312) (end 97.048 98.3) (width 0.254) (layer "F.Cu") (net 8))
 (segment (start 97.048 96.547) (end 98.22 95.375) (width 0.254) (layer "F.Cu") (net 8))
 (segment (start 99.041 99.312) (end 98.061 99.312) (width 0.254) (layer "F.Cu") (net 8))
 (segment (start 99.49 94.105) (end 98.22 92.835) (width 0.254) (layer "F.Cu") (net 9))
 (segment (start 156.64 94.105) (end 99.49 94.105) (width 0.254) (layer "F.Cu") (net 9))
 (via (at 156.64 94.105) (size 0.61) (drill 0.305) (layers "F.Cu" "B.Cu") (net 9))
 (segment (start 167.3 103.5) (end 166.035 103.5) (width 0.254) (layer "B.Cu") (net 9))
 (segment (start 166.035 103.5) (end 156.64 94.105) (width 0.254) (layer "B.Cu") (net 9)))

